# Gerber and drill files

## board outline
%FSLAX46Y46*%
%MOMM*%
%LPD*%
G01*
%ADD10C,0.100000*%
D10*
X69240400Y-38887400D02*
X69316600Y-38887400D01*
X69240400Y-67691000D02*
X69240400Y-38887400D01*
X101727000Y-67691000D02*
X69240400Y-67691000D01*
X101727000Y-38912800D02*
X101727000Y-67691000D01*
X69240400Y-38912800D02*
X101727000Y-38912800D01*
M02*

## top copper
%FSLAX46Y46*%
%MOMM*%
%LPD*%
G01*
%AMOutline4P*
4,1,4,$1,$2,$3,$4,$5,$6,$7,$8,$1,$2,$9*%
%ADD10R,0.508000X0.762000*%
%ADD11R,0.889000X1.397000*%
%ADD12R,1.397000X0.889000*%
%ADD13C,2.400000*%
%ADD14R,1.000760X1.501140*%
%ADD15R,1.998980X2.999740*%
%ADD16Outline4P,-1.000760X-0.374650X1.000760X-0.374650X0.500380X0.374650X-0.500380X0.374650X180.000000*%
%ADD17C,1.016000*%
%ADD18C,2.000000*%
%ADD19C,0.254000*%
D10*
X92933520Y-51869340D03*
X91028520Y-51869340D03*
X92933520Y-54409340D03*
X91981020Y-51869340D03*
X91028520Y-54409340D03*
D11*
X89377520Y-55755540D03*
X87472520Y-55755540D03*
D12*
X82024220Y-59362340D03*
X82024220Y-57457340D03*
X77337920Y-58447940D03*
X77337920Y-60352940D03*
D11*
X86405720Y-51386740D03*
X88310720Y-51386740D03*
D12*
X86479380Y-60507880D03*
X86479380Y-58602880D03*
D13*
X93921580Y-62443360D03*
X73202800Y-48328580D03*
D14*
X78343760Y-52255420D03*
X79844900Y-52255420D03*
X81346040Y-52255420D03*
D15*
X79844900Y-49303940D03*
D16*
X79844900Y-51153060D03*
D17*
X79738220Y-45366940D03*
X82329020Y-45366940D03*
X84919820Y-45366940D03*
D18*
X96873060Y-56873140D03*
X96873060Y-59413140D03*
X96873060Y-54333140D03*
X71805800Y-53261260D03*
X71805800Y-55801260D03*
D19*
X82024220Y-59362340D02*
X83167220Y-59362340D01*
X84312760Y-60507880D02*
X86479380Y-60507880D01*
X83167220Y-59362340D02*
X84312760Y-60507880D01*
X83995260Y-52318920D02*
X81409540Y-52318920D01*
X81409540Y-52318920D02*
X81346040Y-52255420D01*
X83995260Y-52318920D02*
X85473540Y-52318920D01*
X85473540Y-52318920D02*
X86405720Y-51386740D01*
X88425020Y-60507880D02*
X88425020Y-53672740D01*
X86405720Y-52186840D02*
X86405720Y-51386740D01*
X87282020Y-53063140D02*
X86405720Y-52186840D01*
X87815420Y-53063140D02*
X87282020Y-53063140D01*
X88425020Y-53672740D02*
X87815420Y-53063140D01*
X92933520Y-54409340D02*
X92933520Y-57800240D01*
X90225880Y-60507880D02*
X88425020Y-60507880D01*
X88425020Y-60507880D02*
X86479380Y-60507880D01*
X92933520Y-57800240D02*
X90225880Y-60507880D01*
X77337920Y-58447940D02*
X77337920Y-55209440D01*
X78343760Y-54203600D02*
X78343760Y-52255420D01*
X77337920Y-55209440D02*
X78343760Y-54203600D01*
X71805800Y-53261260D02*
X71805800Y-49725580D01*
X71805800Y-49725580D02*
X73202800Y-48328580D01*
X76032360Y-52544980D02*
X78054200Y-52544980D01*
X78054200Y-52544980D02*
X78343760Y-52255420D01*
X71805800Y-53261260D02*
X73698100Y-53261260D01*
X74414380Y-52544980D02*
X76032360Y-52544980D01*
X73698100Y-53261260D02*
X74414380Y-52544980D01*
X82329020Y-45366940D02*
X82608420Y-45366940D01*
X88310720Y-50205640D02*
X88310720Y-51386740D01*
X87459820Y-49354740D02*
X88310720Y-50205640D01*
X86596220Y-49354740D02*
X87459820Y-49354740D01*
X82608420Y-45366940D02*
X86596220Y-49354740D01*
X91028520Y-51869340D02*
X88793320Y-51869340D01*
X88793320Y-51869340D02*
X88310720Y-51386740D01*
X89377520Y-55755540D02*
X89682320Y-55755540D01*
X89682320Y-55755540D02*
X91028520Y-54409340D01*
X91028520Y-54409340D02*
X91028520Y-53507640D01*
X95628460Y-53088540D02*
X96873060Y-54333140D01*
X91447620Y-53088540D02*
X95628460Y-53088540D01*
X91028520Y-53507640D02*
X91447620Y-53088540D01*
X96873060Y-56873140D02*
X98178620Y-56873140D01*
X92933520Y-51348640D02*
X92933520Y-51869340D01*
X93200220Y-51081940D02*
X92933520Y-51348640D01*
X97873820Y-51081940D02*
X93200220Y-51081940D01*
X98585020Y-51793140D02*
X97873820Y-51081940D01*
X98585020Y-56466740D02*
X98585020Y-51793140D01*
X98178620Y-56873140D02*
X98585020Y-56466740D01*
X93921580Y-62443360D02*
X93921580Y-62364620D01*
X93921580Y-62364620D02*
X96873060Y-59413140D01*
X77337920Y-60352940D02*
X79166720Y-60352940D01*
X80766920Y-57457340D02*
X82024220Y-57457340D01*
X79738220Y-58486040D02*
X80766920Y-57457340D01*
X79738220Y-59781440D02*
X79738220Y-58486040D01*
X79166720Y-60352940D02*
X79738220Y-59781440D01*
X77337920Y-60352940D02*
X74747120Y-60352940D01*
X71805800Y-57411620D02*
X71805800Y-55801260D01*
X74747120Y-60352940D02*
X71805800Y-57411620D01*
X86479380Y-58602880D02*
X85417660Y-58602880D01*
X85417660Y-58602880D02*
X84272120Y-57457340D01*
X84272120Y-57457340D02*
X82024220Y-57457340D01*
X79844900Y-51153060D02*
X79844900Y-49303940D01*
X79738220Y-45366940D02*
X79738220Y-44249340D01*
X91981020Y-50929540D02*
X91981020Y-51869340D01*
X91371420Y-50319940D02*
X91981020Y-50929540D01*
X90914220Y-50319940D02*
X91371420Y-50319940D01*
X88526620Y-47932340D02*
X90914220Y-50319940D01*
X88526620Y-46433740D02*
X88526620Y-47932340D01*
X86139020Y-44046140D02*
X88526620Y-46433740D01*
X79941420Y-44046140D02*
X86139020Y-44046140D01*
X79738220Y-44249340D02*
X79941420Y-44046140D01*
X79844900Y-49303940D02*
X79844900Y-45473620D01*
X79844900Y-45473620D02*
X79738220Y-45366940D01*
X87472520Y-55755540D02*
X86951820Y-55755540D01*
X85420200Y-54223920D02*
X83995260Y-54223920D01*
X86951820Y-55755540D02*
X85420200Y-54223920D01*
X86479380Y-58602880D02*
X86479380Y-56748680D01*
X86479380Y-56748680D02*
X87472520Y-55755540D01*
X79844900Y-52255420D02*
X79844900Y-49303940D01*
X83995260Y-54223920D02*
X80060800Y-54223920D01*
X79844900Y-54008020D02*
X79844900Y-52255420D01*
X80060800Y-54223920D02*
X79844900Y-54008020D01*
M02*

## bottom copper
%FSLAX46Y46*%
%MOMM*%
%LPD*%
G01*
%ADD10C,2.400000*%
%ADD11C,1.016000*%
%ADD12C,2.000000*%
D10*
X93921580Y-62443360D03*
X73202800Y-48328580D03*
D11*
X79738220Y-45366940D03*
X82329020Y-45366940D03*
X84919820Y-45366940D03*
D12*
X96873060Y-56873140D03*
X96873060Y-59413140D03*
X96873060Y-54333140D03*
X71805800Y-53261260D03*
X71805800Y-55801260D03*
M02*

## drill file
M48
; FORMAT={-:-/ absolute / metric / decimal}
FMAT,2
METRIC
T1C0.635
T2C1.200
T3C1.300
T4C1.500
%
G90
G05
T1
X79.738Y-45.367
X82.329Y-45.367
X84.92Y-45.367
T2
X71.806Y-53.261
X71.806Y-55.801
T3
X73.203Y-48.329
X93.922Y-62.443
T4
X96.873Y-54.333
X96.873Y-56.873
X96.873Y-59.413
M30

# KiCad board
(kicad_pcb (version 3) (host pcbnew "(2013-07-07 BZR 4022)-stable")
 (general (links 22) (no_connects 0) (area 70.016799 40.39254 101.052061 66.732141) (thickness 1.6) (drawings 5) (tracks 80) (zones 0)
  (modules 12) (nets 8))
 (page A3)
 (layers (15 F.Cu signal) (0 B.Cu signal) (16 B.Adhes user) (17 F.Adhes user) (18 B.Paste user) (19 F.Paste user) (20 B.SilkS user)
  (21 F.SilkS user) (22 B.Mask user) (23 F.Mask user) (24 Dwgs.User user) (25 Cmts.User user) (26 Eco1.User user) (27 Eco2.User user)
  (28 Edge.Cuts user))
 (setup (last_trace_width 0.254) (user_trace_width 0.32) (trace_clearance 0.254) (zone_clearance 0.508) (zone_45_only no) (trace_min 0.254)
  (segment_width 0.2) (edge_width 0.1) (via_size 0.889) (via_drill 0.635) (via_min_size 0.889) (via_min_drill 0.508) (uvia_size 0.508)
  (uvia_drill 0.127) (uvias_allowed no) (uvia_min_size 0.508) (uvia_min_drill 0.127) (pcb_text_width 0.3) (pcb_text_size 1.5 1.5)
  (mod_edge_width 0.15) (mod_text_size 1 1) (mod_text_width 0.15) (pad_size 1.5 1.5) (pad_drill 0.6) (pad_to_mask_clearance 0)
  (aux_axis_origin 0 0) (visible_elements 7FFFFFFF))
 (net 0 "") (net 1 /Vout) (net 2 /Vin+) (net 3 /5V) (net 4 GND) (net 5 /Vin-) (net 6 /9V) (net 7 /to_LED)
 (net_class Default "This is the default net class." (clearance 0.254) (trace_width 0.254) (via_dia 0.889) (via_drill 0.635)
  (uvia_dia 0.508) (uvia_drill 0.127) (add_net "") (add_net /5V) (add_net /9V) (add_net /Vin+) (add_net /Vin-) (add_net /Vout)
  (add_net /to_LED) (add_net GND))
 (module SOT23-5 (layer F.Cu) (at 91.98102 53.13934 180)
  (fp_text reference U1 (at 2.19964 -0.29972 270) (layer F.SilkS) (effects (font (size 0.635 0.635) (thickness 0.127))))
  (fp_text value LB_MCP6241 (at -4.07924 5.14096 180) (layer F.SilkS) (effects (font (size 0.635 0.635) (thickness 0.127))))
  (pad 1 smd rect (at -0.9525 1.27 180) (size 0.508 0.762) (layers F.Cu F.Paste F.Mask) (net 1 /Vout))
  (pad 3 smd rect (at 0.9525 1.27 180) (size 0.508 0.762) (layers F.Cu F.Paste F.Mask) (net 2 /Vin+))
  (pad 5 smd rect (at -0.9525 -1.27 180) (size 0.508 0.762) (layers F.Cu F.Paste F.Mask) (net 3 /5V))
  (pad 2 smd rect (at 0 1.27 180) (size 0.508 0.762) (layers F.Cu F.Paste F.Mask) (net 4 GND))
  (pad 4 smd rect (at 0.9525 -1.27 180) (size 0.508 0.762) (layers F.Cu F.Paste F.Mask) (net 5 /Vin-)))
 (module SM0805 (layer F.Cu) (at 88.42502 55.75554 180)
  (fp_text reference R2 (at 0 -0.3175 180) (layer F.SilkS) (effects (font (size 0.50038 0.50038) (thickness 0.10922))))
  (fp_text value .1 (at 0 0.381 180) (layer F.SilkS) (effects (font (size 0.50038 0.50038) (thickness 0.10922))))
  (pad 1 smd rect (at -0.9525 0 180) (size 0.889 1.397) (layers F.Cu F.Paste F.Mask) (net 5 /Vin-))
  (pad 2 smd rect (at 0.9525 0 180) (size 0.889 1.397) (layers F.Cu F.Paste F.Mask) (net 4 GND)))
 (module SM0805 (layer F.Cu) (at 82.02422 58.40984 90)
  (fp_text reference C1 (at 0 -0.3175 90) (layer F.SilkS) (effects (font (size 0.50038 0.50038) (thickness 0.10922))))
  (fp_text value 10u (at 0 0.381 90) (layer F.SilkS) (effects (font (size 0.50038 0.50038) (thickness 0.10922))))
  (pad 1 smd rect (at -0.9525 0 90) (size 0.889 1.397) (layers F.Cu F.Paste F.Mask) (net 3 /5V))
  (pad 2 smd rect (at 0.9525 0 90) (size 0.889 1.397) (layers F.Cu F.Paste F.Mask) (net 4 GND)))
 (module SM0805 (layer F.Cu) (at 77.33792 59.40044 270)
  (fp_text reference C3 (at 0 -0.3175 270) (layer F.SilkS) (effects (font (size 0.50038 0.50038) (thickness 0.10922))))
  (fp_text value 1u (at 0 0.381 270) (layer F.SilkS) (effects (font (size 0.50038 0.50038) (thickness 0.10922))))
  (pad 1 smd rect (at -0.9525 0 270) (size 0.889 1.397) (layers F.Cu F.Paste F.Mask) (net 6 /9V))
  (pad 2 smd rect (at 0.9525 0 270) (size 0.889 1.397) (layers F.Cu F.Paste F.Mask) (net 4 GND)))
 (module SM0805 (layer F.Cu) (at 87.35822 51.38674)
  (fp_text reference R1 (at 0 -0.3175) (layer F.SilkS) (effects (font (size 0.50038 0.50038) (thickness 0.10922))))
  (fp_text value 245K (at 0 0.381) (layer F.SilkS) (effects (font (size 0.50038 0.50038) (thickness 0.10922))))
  (pad 1 smd rect (at -0.9525 0) (size 0.889 1.397) (layers F.Cu F.Paste F.Mask) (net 3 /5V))
  (pad 2 smd rect (at 0.9525 0) (size 0.889 1.397) (layers F.Cu F.Paste F.Mask) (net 2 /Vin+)))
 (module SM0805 (layer F.Cu) (at 86.47938 59.55538 90)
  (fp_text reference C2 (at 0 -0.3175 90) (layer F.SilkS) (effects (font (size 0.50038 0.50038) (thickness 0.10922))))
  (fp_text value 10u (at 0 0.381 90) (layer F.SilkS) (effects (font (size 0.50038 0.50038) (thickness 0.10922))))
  (pad 1 smd rect (at -0.9525 0 90) (size 0.889 1.397) (layers F.Cu F.Paste F.Mask) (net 3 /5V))
  (pad 2 smd rect (at 0.9525 0 90) (size 0.889 1.397) (layers F.Cu F.Paste F.Mask) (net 4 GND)))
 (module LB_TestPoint (layer F.Cu) (at 93.92158 62.44336)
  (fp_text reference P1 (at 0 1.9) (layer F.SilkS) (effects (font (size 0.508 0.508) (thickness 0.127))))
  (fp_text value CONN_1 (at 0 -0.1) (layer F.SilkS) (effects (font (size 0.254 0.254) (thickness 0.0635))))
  (pad 1 thru_hole circle (at 0 0) (size 2.4 2.4) (drill 1.3) (layers *.Cu *.Mask F.SilkS) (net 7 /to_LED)))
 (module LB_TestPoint (layer F.Cu) (at 73.2028 48.32858)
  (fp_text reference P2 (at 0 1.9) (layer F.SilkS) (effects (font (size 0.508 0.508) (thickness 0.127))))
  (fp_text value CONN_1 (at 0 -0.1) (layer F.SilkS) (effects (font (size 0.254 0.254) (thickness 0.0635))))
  (pad 1 thru_hole circle (at 0 0) (size 2.4 2.4) (drill 1.3) (layers *.Cu *.Mask F.SilkS) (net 6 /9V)))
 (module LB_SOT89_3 (layer F.Cu) (at 79.8449 50.40376)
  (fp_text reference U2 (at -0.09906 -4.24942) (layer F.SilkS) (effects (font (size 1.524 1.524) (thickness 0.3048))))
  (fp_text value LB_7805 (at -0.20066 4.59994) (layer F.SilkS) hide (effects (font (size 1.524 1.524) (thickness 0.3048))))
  (pad 1 smd rect (at -1.50114 1.85166) (size 1.00076 1.50114) (layers F.Cu F.Paste F.Mask) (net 6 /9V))
  (pad 2 smd rect (at 0 1.85166) (size 1.00076 1.50114) (layers F.Cu F.Paste F.Mask) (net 4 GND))
  (pad 3 smd rect (at 1.50114 1.85166) (size 1.00076 1.50114) (layers F.Cu F.Paste F.Mask) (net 3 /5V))
  (pad 2 smd rect (at 0 -1.09982) (size 1.99898 2.99974) (layers F.Cu F.Paste F.Mask) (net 4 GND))
  (pad 2 smd trapezoid (at 0 0.7493 180) (size 1.50114 0.7493) (rect_delta 0 0.50038) (layers F.Cu F.Paste F.Mask) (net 4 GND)))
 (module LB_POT (layer F.Cu) (at 77.50302 40.89654)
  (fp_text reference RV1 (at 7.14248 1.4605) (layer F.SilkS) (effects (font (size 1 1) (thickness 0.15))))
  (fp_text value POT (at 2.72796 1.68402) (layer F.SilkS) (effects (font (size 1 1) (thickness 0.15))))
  (pad 1 thru_hole circle (at 2.2352 4.4704) (size 1.016 1.016) (drill 0.635) (layers *.Cu *.Mask F.SilkS) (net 4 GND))
  (pad 2 thru_hole circle (at 4.826 4.4704) (size 1.016 1.016) (drill 0.635) (layers *.Cu *.Mask F.SilkS) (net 2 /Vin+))
  (pad 3 thru_hole circle (at 7.4168 4.4704) (size 1.016 1.016) (drill 0.635) (layers *.Cu *.Mask F.SilkS)))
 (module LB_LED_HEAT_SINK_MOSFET (layer F.Cu) (at 96.87306 56.87314 270)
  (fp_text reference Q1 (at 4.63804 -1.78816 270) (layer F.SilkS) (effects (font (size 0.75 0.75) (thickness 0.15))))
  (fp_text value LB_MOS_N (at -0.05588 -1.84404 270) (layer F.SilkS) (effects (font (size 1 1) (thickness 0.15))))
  (pad 1 thru_hole circle (at 0 0 270) (size 2 2) (drill 1.5) (layers *.Cu *.Mask F.SilkS) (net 1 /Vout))
  (pad 2 thru_hole circle (at 2.54 0 270) (size 2 2) (drill 1.5) (layers *.Cu *.Mask F.SilkS) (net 7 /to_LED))
  (pad 3 thru_hole circle (at -2.54 0 270) (size 2 2) (drill 1.5) (layers *.Cu *.Mask F.SilkS) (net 5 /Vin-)))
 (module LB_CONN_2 (layer F.Cu) (at 71.8058 55.80126 270)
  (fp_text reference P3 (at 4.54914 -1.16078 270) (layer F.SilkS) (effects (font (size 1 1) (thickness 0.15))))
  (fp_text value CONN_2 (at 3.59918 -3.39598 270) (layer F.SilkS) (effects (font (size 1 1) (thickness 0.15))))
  (pad 1 thru_hole circle (at -2.54 0 270) (size 2 2) (drill 1.2) (layers *.Cu *.Mask F.SilkS) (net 6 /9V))
  (pad 2 thru_hole circle (at 0 0 270) (size 2 2) (drill 1.2) (layers *.Cu *.Mask F.SilkS) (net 4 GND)))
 (gr_line (start 69.2404 38.8874) (end 69.3166 38.8874) (angle 90) (layer Edge.Cuts) (width 0.1))
 (gr_line (start 69.2404 67.691) (end 69.2404 38.8874) (angle 90) (layer Edge.Cuts) (width 0.1))
 (gr_line (start 101.727 67.691) (end 69.2404 67.691) (angle 90) (layer Edge.Cuts) (width 0.1))
 (gr_line (start 101.727 38.9128) (end 101.727 67.691) (angle 90) (layer Edge.Cuts) (width 0.1))
 (gr_line (start 69.2404 38.9128) (end 101.727 38.9128) (angle 90) (layer Edge.Cuts) (width 0.1))
 (segment (start 82.02422 59.36234) (end 83.16722 59.36234) (width 0.254) (layer F.Cu) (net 3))
 (segment (start 84.31276 60.50788) (end 86.47938 60.50788) (width 0.254) (layer F.Cu) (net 3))
 (segment (start 83.16722 59.36234) (end 84.31276 60.50788) (width 0.254) (layer F.Cu) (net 3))
 (segment (start 83.99526 52.31892) (end 81.40954 52.31892) (width 0.254) (layer F.Cu) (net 3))
 (segment (start 81.40954 52.31892) (end 81.34604 52.25542) (width 0.254) (layer F.Cu) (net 3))
 (segment (start 83.99526 52.31892) (end 85.47354 52.31892) (width 0.254) (layer F.Cu) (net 3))
 (segment (start 85.47354 52.31892) (end 86.40572 51.38674) (width 0.254) (layer F.Cu) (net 3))
 (segment (start 88.42502 60.50788) (end 88.42502 53.67274) (width 0.254) (layer F.Cu) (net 3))
 (segment (start 86.40572 52.18684) (end 86.40572 51.38674) (width 0.254) (layer F.Cu) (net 3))
 (segment (start 87.28202 53.06314) (end 86.40572 52.18684) (width 0.254) (layer F.Cu) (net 3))
 (segment (start 87.81542 53.06314) (end 87.28202 53.06314) (width 0.254) (layer F.Cu) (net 3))
 (segment (start 88.42502 53.67274) (end 87.81542 53.06314) (width 0.254) (layer F.Cu) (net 3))
 (segment (start 92.93352 54.40934) (end 92.93352 57.80024) (width 0.254) (layer F.Cu) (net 3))
 (segment (start 90.22588 60.50788) (end 88.42502 60.50788) (width 0.254) (layer F.Cu) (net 3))
 (segment (start 88.42502 60.50788) (end 86.47938 60.50788) (width 0.254) (layer F.Cu) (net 3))
 (segment (start 92.93352 57.80024) (end 90.22588 60.50788) (width 0.254) (layer F.Cu) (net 3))
 (segment (start 77.33792 58.44794) (end 77.33792 55.20944) (width 0.254) (layer F.Cu) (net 6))
 (segment (start 78.34376 54.2036) (end 78.34376 52.25542) (width 0.254) (layer F.Cu) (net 6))
 (segment (start 77.33792 55.20944) (end 78.34376 54.2036) (width 0.254) (layer F.Cu) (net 6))
 (segment (start 71.8058 53.26126) (end 71.8058 49.72558) (width 0.254) (layer F.Cu) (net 6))
 (segment (start 71.8058 49.72558) (end 73.2028 48.32858) (width 0.254) (layer F.Cu) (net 6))
 (segment (start 76.03236 52.54498) (end 78.0542 52.54498) (width 0.254) (layer F.Cu) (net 6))
 (segment (start 78.0542 52.54498) (end 78.34376 52.25542) (width 0.254) (layer F.Cu) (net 6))
 (segment (start 71.8058 53.26126) (end 73.6981 53.26126) (width 0.254) (layer F.Cu) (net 6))
 (segment (start 74.41438 52.54498) (end 76.03236 52.54498) (width 0.254) (layer F.Cu) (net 6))
 (segment (start 73.6981 53.26126) (end 74.41438 52.54498) (width 0.254) (layer F.Cu) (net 6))
 (segment (start 82.32902 45.36694) (end 82.60842 45.36694) (width 0.254) (layer F.Cu) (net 2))
 (segment (start 88.31072 50.20564) (end 88.31072 51.38674) (width 0.254) (layer F.Cu) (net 2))
 (segment (start 87.45982 49.35474) (end 88.31072 50.20564) (width 0.254) (layer F.Cu) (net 2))
 (segment (start 86.59622 49.35474) (end 87.45982 49.35474) (width 0.254) (layer F.Cu) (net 2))
 (segment (start 82.60842 45.36694) (end 86.59622 49.35474) (width 0.254) (layer F.Cu) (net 2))
 (segment (start 91.02852 51.86934) (end 88.79332 51.86934) (width 0.254) (layer F.Cu) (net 2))
 (segment (start 88.79332 51.86934) (end 88.31072 51.38674) (width 0.254) (layer F.Cu) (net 2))
 (segment (start 89.37752 55.75554) (end 89.68232 55.75554) (width 0.254) (layer F.Cu) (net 5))
 (segment (start 89.68232 55.75554) (end 91.02852 54.40934) (width 0.254) (layer F.Cu) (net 5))
 (segment (start 91.02852 54.40934) (end 91.02852 53.50764) (width 0.254) (layer F.Cu) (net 5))
 (segment (start 95.62846 53.08854) (end 96.87306 54.33314) (width 0.254) (layer F.Cu) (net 5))
 (segment (start 91.44762 53.08854) (end 95.62846 53.08854) (width 0.254) (layer F.Cu) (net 5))
 (segment (start 91.02852 53.50764) (end 91.44762 53.08854) (width 0.254) (layer F.Cu) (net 5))
 (segment (start 96.87306 56.87314) (end 98.17862 56.87314) (width 0.254) (layer F.Cu) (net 1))
 (segment (start 92.93352 51.34864) (end 92.93352 51.86934) (width 0.254) (layer F.Cu) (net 1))
 (segment (start 93.20022 51.08194) (end 92.93352 51.34864) (width 0.254) (layer F.Cu) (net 1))
 (segment (start 97.87382 51.08194) (end 93.20022 51.08194) (width 0.254) (layer F.Cu) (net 1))
 (segment (start 98.58502 51.79314) (end 97.87382 51.08194) (width 0.254) (layer F.Cu) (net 1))
 (segment (start 98.58502 56.46674) (end 98.58502 51.79314) (width 0.254) (layer F.Cu) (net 1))
 (segment (start 98.17862 56.87314) (end 98.58502 56.46674) (width 0.254) (layer F.Cu) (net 1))
 (segment (start 93.92158 62.44336) (end 93.92158 62.36462) (width 0.254) (layer F.Cu) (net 7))
 (segment (start 93.92158 62.36462) (end 96.87306 59.41314) (width 0.254) (layer F.Cu) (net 7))
 (segment (start 77.33792 60.35294) (end 79.16672 60.35294) (width 0.254) (layer F.Cu) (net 4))
 (segment (start 80.76692 57.45734) (end 82.02422 57.45734) (width 0.254) (layer F.Cu) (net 4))
 (segment (start 79.73822 58.48604) (end 80.76692 57.45734) (width 0.254) (layer F.Cu) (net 4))
 (segment (start 79.73822 59.78144) (end 79.73822 58.48604) (width 0.254) (layer F.Cu) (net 4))
 (segment (start 79.16672 60.35294) (end 79.73822 59.78144) (width 0.254) (layer F.Cu) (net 4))
 (segment (start 77.33792 60.35294) (end 74.74712 60.35294) (width 0.254) (layer F.Cu) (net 4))
 (segment (start 71.8058 57.41162) (end 71.8058 55.80126) (width 0.254) (layer F.Cu) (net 4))
 (segment (start 74.74712 60.35294) (end 71.8058 57.41162) (width 0.254) (layer F.Cu) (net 4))
 (segment (start 86.47938 58.60288) (end 85.41766 58.60288) (width 0.254) (layer F.Cu) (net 4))
 (segment (start 85.41766 58.60288) (end 84.27212 57.45734) (width 0.254) (layer F.Cu) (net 4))
 (segment (start 84.27212 57.45734) (end 82.02422 57.45734) (width 0.254) (layer F.Cu) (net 4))
 (segment (start 79.8449 51.15306) (end 79.8449 49.30394) (width 0.254) (layer F.Cu) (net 4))
 (segment (start 79.73822 45.36694) (end 79.73822 44.24934) (width 0.254) (layer F.Cu) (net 4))
 (segment (start 91.98102 50.92954) (end 91.98102 51.86934) (width 0.254) (layer F.Cu) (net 4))
 (segment (start 91.37142 50.31994) (end 91.98102 50.92954) (width 0.254) (layer F.Cu) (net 4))
 (segment (start 90.91422 50.31994) (end 91.37142 50.31994) (width 0.254) (layer F.Cu) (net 4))
 (segment (start 88.52662 47.93234) (end 90.91422 50.31994) (width 0.254) (layer F.Cu) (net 4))
 (segment (start 88.52662 46.43374) (end 88.52662 47.93234) (width 0.254) (layer F.Cu) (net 4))
 (segment (start 86.13902 44.04614) (end 88.52662 46.43374) (width 0.254) (layer F.Cu) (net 4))
 (segment (start 79.94142 44.04614) (end 86.13902 44.04614) (width 0.254) (layer F.Cu) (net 4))
 (segment (start 79.73822 44.24934) (end 79.94142 44.04614) (width 0.254) (layer F.Cu) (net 4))
 (segment (start 79.8449 49.30394) (end 79.8449 45.47362) (width 0.254) (layer F.Cu) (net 4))
 (segment (start 79.8449 45.47362) (end 79.73822 45.36694) (width 0.254) (layer F.Cu) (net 4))
 (segment (start 87.47252 55.75554) (end 86.95182 55.75554) (width 0.254) (layer F.Cu) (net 4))
 (segment (start 85.4202 54.22392) (end 83.99526 54.22392) (width 0.254) (layer F.Cu) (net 4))
 (segment (start 86.95182 55.75554) (end 85.4202 54.22392) (width 0.254) (layer F.Cu) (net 4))
 (segment (start 86.47938 58.60288) (end 86.47938 56.74868) (width 0.254) (layer F.Cu) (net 4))
 (segment (start 86.47938 56.74868) (end 87.47252 55.75554) (width 0.254) (layer F.Cu) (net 4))
 (segment (start 79.8449 52.25542) (end 79.8449 49.30394) (width 0.254) (layer F.Cu) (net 4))
 (segment (start 83.99526 54.22392) (end 80.0608 54.22392) (width 0.254) (layer F.Cu) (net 4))
 (segment (start 79.8449 54.00802) (end 79.8449 52.25542) (width 0.254) (layer F.Cu) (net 4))
 (segment (start 80.0608 54.22392) (end 79.8449 54.00802) (width 0.254) (layer F.Cu) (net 4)))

